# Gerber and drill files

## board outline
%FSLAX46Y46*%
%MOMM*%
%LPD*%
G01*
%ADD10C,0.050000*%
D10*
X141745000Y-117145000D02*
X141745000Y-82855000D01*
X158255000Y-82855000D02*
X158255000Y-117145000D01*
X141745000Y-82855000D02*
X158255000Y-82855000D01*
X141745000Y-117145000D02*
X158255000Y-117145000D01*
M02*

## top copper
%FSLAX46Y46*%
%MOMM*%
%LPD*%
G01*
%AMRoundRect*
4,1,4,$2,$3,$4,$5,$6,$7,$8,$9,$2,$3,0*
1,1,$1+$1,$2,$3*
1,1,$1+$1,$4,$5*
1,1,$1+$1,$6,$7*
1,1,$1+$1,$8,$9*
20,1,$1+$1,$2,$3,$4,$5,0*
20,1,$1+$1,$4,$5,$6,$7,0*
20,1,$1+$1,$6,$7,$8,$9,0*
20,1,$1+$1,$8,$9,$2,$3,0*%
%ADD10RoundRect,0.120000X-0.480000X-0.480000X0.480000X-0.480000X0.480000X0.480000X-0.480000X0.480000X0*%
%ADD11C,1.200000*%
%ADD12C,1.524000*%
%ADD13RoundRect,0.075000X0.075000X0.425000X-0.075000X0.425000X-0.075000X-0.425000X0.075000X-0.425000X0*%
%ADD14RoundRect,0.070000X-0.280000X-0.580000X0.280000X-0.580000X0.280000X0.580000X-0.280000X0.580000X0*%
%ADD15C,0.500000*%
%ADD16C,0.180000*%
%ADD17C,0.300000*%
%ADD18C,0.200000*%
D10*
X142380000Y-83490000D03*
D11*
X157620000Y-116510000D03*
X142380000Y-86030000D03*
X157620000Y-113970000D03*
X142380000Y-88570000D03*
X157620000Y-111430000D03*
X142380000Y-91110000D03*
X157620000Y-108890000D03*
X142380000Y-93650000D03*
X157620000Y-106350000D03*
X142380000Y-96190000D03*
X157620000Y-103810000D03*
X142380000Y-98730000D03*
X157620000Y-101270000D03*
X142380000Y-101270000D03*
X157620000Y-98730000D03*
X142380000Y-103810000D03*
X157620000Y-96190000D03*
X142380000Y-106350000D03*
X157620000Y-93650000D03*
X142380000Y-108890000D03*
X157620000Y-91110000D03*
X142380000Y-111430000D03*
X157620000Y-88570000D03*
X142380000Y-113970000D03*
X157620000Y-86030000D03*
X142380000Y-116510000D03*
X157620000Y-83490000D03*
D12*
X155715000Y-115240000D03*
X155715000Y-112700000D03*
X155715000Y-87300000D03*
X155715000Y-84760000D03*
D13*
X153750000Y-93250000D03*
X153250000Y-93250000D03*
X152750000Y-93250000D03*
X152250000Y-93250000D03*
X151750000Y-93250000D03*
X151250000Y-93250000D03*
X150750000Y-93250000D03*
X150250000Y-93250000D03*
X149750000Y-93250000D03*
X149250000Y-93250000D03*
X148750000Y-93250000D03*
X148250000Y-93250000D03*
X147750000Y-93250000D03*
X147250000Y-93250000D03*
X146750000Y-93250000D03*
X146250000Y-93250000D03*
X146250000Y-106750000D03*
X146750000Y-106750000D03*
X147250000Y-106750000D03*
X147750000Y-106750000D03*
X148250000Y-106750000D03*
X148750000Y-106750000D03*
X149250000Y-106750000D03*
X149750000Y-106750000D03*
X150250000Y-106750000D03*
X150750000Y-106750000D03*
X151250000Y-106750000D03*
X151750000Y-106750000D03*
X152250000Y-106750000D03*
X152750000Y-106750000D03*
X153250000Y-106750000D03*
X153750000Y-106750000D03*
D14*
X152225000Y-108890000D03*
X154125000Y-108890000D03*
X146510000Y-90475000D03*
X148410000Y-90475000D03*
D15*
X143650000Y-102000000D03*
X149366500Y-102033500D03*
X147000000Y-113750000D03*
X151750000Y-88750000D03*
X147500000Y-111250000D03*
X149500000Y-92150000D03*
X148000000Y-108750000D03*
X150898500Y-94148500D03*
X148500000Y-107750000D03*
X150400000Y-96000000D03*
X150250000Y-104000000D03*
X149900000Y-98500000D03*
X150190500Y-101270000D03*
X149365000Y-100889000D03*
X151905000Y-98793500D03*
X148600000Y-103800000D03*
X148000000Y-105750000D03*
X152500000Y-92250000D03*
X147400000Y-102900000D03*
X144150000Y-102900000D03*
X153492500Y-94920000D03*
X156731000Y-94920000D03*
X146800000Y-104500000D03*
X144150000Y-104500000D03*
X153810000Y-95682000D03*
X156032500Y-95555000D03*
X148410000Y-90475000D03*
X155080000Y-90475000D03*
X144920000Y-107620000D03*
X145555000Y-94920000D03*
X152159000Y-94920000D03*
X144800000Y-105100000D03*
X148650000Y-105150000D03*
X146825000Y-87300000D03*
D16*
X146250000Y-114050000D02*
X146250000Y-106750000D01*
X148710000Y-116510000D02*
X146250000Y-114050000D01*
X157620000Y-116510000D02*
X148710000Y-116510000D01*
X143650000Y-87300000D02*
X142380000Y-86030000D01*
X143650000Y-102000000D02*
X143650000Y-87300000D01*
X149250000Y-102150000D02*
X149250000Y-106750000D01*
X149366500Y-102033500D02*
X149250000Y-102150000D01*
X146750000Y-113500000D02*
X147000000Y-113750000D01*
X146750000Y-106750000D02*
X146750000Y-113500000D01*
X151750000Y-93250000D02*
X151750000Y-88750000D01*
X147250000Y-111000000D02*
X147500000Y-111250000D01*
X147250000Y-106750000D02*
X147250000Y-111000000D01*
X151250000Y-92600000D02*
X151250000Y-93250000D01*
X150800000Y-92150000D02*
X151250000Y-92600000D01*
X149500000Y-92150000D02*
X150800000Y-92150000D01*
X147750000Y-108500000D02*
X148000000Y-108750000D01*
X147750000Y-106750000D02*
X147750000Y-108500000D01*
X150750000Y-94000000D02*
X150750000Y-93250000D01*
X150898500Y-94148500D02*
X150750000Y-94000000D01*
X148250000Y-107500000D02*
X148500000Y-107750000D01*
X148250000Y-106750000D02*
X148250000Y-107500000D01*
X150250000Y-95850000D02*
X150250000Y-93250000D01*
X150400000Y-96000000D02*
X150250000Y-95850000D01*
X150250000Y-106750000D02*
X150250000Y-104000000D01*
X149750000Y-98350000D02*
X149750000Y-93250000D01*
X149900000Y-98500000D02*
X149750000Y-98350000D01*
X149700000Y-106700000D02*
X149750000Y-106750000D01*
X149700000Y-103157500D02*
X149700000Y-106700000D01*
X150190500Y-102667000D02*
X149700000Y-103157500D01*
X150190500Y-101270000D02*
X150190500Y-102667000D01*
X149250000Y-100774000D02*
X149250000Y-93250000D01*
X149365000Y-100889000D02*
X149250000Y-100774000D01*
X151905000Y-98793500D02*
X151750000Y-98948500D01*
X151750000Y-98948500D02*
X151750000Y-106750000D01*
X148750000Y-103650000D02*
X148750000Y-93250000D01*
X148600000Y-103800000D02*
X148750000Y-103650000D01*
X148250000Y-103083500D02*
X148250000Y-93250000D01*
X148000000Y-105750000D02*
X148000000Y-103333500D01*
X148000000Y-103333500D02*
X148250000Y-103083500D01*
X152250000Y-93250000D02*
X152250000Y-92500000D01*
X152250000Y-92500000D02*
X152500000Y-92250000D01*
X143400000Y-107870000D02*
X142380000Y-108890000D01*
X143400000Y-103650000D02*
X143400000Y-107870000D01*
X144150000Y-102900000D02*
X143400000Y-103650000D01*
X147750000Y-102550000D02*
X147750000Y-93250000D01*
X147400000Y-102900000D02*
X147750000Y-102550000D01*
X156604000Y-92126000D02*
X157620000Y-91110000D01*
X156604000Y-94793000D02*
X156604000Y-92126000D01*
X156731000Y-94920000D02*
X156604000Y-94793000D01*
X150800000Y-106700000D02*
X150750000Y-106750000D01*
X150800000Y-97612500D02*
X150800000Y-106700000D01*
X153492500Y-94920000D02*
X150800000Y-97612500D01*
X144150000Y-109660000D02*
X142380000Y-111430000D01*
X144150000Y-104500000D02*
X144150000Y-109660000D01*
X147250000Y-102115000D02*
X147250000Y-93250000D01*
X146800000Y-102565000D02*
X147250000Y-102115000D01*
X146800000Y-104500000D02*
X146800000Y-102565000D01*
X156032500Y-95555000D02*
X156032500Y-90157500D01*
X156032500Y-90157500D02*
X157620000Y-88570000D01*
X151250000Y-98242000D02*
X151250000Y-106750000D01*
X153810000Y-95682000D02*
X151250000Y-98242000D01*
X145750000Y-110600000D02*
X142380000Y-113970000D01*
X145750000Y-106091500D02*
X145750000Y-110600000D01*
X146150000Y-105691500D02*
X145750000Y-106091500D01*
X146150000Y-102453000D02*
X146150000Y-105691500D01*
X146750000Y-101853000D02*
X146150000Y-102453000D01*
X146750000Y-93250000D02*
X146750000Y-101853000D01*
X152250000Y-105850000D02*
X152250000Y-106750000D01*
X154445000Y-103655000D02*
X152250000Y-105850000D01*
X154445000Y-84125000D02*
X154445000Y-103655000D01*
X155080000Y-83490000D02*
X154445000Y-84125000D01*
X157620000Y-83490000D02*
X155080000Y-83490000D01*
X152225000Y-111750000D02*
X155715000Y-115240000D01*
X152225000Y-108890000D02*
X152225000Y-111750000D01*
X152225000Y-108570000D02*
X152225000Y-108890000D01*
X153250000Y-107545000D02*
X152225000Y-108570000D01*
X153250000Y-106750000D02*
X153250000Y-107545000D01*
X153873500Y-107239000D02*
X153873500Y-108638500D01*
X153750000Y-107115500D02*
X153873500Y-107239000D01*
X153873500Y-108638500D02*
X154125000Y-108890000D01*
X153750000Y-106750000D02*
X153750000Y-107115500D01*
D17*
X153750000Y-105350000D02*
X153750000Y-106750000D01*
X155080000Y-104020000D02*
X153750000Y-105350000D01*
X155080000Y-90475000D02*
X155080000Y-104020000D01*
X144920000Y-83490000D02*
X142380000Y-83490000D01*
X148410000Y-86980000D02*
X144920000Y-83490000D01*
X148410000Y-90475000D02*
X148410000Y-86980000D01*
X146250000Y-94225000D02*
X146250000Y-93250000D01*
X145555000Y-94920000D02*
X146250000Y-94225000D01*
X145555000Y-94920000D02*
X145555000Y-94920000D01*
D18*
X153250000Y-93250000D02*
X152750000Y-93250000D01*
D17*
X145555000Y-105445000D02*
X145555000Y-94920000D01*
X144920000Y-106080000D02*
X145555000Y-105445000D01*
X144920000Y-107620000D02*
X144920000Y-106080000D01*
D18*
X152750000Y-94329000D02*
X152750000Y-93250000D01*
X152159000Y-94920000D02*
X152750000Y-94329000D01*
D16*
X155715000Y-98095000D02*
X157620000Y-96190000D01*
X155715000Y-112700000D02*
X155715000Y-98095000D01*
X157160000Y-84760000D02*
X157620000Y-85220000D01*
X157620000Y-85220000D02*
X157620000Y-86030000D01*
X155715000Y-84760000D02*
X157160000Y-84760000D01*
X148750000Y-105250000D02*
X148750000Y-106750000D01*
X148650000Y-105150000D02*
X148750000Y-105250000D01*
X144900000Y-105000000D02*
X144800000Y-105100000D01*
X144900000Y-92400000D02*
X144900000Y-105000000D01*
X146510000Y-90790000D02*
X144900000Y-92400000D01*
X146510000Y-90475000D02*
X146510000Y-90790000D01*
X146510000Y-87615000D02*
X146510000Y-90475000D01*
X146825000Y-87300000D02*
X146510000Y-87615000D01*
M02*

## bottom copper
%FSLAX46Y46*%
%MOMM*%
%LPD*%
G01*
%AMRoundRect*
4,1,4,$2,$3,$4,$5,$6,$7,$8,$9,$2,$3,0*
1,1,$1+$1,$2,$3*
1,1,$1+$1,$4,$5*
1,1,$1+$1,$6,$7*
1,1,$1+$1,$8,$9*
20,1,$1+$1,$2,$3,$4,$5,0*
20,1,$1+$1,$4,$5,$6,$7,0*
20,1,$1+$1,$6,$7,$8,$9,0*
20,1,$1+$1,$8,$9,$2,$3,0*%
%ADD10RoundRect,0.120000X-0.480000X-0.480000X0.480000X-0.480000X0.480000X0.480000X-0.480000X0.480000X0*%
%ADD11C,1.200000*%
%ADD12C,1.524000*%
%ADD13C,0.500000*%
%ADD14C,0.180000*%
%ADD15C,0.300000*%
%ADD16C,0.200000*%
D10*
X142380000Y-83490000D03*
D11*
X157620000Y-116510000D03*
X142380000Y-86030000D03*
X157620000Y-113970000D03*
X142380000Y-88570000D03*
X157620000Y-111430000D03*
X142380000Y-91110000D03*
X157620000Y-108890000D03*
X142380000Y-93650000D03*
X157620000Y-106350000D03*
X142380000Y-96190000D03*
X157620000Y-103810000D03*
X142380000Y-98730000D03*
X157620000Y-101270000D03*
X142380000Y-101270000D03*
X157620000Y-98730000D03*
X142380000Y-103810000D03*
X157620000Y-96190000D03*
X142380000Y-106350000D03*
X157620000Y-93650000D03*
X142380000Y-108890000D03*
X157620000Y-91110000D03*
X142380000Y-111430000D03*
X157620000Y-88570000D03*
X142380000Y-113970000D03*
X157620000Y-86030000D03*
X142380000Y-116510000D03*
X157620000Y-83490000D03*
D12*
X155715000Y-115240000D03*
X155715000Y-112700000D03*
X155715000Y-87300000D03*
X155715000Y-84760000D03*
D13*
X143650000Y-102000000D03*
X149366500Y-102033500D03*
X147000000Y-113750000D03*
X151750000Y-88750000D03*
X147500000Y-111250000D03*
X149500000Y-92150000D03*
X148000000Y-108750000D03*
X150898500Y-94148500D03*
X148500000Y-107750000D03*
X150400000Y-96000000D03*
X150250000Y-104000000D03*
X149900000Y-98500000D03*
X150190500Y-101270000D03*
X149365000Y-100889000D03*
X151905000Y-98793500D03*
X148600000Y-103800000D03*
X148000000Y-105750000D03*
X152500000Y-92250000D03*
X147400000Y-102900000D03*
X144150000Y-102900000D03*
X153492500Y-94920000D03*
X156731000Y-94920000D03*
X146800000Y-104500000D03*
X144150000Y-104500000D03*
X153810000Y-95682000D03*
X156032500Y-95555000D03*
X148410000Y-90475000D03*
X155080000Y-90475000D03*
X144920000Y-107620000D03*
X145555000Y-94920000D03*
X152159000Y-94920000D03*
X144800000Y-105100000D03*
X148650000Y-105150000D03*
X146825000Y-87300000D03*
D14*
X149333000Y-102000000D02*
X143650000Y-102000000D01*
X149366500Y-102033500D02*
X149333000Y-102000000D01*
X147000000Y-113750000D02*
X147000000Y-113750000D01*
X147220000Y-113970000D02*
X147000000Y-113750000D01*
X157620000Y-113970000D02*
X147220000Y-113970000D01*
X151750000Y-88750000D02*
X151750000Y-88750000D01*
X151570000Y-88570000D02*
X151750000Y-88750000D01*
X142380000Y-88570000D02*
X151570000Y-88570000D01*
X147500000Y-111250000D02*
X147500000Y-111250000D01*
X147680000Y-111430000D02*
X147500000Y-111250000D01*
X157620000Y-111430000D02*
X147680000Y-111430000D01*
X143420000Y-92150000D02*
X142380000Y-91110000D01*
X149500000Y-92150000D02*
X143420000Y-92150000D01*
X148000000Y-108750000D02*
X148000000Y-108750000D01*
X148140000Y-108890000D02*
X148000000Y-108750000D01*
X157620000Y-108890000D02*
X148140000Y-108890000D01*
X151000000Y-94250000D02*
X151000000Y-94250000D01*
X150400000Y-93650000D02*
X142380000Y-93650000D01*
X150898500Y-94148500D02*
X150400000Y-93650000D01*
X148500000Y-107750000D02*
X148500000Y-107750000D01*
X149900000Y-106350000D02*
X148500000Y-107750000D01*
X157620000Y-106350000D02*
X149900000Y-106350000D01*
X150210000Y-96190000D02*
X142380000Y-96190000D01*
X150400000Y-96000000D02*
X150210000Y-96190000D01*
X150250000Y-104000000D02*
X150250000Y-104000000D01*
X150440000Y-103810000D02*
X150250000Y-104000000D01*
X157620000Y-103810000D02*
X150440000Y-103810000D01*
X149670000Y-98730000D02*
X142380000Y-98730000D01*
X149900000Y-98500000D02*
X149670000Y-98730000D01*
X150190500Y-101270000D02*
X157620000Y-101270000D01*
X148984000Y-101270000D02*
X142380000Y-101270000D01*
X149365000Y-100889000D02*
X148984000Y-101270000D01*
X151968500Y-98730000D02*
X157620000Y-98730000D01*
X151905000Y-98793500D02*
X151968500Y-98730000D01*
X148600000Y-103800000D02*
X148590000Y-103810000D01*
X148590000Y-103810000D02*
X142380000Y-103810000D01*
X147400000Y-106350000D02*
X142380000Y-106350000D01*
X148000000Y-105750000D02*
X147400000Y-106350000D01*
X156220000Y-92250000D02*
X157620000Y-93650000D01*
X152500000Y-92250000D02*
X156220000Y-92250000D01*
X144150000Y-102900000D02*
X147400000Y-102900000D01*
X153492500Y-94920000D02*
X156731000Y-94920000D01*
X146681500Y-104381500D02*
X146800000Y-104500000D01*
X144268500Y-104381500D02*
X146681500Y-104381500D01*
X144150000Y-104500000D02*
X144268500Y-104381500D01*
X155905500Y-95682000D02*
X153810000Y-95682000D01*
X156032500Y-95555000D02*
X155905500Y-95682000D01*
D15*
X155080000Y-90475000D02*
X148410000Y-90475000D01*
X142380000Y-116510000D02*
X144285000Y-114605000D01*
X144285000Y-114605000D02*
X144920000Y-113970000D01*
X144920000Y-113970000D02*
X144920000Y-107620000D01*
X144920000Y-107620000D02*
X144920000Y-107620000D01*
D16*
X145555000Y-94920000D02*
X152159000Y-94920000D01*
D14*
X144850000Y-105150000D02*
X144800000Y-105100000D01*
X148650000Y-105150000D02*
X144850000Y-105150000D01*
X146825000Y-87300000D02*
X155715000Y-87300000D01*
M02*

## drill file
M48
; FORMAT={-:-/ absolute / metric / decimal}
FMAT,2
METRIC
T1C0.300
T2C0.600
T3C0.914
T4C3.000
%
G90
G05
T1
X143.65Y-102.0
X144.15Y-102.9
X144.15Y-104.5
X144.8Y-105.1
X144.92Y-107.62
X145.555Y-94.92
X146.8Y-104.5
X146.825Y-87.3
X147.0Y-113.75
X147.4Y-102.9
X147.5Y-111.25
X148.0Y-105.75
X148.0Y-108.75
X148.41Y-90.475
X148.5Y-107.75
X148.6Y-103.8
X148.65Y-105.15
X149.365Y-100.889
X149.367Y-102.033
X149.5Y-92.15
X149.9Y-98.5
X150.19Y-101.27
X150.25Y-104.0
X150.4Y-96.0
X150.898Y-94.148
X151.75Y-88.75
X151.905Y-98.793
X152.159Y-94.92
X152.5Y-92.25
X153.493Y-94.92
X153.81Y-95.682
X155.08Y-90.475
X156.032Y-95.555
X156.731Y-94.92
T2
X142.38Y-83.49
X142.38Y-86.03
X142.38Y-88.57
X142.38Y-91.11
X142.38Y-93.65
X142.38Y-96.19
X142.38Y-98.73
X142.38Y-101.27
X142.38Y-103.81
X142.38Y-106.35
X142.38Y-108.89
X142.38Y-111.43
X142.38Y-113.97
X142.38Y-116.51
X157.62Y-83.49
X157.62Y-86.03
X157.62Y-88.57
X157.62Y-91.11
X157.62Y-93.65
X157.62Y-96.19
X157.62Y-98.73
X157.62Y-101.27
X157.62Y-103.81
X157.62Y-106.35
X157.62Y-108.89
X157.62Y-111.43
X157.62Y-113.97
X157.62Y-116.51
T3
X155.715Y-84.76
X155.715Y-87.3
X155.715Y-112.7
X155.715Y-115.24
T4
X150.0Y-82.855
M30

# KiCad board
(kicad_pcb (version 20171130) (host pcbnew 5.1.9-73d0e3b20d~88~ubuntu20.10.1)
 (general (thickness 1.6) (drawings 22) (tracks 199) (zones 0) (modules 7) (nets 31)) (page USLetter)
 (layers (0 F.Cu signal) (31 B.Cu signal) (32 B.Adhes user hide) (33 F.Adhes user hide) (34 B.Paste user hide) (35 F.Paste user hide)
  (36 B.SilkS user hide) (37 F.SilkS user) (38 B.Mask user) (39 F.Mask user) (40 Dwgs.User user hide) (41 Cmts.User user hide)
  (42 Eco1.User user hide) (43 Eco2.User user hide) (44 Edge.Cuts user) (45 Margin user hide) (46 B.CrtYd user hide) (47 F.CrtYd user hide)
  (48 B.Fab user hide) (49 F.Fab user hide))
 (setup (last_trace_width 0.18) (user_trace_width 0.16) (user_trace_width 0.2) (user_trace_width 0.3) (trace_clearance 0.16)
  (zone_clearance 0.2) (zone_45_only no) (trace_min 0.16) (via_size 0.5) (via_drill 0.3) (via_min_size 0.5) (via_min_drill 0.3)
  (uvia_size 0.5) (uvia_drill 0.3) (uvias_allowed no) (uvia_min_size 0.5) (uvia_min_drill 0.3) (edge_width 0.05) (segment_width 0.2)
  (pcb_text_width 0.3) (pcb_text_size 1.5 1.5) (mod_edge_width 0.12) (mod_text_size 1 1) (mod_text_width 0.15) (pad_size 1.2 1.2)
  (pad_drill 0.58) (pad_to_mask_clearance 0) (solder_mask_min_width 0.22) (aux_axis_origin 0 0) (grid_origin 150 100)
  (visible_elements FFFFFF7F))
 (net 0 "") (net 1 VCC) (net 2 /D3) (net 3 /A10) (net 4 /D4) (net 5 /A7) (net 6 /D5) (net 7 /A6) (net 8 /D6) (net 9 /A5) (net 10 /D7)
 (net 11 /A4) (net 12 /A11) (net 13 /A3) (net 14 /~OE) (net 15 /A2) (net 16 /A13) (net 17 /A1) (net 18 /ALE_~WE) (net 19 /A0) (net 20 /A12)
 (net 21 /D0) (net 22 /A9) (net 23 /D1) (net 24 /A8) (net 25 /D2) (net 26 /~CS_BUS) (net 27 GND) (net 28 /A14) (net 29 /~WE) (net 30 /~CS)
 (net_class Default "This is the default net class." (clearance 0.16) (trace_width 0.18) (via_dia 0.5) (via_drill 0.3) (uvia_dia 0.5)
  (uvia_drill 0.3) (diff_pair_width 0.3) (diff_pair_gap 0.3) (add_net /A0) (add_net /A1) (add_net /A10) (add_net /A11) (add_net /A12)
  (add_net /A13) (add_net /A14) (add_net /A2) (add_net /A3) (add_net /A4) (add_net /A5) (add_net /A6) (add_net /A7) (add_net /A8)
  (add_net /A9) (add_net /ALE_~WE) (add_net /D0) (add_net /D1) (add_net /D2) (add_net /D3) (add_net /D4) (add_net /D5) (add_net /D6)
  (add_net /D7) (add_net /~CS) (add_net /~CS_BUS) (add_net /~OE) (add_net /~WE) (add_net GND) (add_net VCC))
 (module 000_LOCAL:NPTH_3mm (layer F.Cu) (at 150 82.855)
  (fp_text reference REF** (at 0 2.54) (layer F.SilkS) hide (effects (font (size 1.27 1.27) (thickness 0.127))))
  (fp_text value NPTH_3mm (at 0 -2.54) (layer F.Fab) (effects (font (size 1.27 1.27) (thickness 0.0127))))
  (pad "" np_thru_hole circle (at 0 0) (size 3 3) (drill 3) (layers *.Cu *.Mask)))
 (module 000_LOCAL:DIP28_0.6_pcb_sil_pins (layer F.Cu) (at 150 100)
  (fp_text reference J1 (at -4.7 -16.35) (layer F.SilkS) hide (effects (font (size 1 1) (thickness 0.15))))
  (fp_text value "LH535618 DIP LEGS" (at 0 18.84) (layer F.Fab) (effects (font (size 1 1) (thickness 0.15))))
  (pad 1 thru_hole roundrect (at -7.62 -16.51) (size 1.2 1.2) (drill 0.6) (layers *.Cu *.Mask) (roundrect_rratio 0.1) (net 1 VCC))
  (pad 15 thru_hole circle (at 7.62 16.51) (size 1.2 1.2) (drill 0.6) (layers *.Cu *.Mask) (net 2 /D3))
  (pad 2 thru_hole circle (at -7.62 -13.97) (size 1.2 1.2) (drill 0.6) (layers *.Cu *.Mask) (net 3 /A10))
  (pad 16 thru_hole circle (at 7.62 13.97) (size 1.2 1.2) (drill 0.6) (layers *.Cu *.Mask) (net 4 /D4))
  (pad 3 thru_hole circle (at -7.62 -11.43) (size 1.2 1.2) (drill 0.6) (layers *.Cu *.Mask) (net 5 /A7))
  (pad 17 thru_hole circle (at 7.62 11.43) (size 1.2 1.2) (drill 0.6) (layers *.Cu *.Mask) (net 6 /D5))
  (pad 4 thru_hole circle (at -7.62 -8.89) (size 1.2 1.2) (drill 0.6) (layers *.Cu *.Mask) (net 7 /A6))
  (pad 18 thru_hole circle (at 7.62 8.89) (size 1.2 1.2) (drill 0.6) (layers *.Cu *.Mask) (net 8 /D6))
  (pad 5 thru_hole circle (at -7.62 -6.35) (size 1.2 1.2) (drill 0.6) (layers *.Cu *.Mask) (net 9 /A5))
  (pad 19 thru_hole circle (at 7.62 6.35) (size 1.2 1.2) (drill 0.6) (layers *.Cu *.Mask) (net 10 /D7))
  (pad 6 thru_hole circle (at -7.62 -3.81) (size 1.2 1.2) (drill 0.6) (layers *.Cu *.Mask) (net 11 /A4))
  (pad 20 thru_hole circle (at 7.62 3.81) (size 1.2 1.2) (drill 0.6) (layers *.Cu *.Mask) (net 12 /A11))
  (pad 7 thru_hole circle (at -7.62 -1.27) (size 1.2 1.2) (drill 0.6) (layers *.Cu *.Mask) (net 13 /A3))
  (pad 21 thru_hole circle (at 7.62 1.27) (size 1.2 1.2) (drill 0.6) (layers *.Cu *.Mask) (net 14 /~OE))
  (pad 8 thru_hole circle (at -7.62 1.27) (size 1.2 1.2) (drill 0.6) (layers *.Cu *.Mask) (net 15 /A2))
  (pad 22 thru_hole circle (at 7.62 -1.27) (size 1.2 1.2) (drill 0.6) (layers *.Cu *.Mask) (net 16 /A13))
  (pad 9 thru_hole circle (at -7.62 3.81) (size 1.2 1.2) (drill 0.6) (layers *.Cu *.Mask) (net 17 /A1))
  (pad 23 thru_hole circle (at 7.62 -3.81) (size 1.2 1.2) (drill 0.6) (layers *.Cu *.Mask) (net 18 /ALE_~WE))
  (pad 10 thru_hole circle (at -7.62 6.35) (size 1.2 1.2) (drill 0.6) (layers *.Cu *.Mask) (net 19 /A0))
  (pad 24 thru_hole circle (at 7.62 -6.35) (size 1.2 1.2) (drill 0.6) (layers *.Cu *.Mask) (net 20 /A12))
  (pad 11 thru_hole circle (at -7.62 8.89) (size 1.2 1.2) (drill 0.6) (layers *.Cu *.Mask) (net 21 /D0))
  (pad 25 thru_hole circle (at 7.62 -8.89) (size 1.2 1.2) (drill 0.6) (layers *.Cu *.Mask) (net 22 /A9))
  (pad 12 thru_hole circle (at -7.62 11.43) (size 1.2 1.2) (drill 0.6) (layers *.Cu *.Mask) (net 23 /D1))
  (pad 26 thru_hole circle (at 7.62 -11.43) (size 1.2 1.2) (drill 0.6) (layers *.Cu *.Mask) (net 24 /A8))
  (pad 13 thru_hole circle (at -7.62 13.97) (size 1.2 1.2) (drill 0.6) (layers *.Cu *.Mask) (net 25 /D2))
  (pad 27 thru_hole circle (at 7.62 -13.97) (size 1.2 1.2) (drill 0.6) (layers *.Cu *.Mask) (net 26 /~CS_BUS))
  (pad 14 thru_hole circle (at -7.62 16.51) (size 1.2 1.2) (drill 0.6) (layers *.Cu *.Mask) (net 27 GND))
  (pad 28 thru_hole circle (at 7.62 -16.51) (size 1.2 1.2) (drill 0.6) (layers *.Cu *.Mask) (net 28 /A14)))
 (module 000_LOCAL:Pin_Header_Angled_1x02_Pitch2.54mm (layer F.Cu) (at 155.715 115.24 180)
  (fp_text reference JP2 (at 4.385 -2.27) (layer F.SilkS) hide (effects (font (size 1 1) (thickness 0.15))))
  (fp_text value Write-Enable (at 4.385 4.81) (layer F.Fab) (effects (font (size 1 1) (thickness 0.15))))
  (pad 1 thru_hole circle (at 0 0 180) (size 1.524 1.524) (drill 0.9144) (layers *.Cu *.Mask) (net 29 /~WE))
  (pad 2 thru_hole circle (at 0 2.54 180) (size 1.524 1.524) (drill 0.9144) (layers *.Cu *.Mask) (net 18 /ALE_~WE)))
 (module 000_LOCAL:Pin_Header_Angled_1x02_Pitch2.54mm (layer F.Cu) (at 155.715 87.3 180)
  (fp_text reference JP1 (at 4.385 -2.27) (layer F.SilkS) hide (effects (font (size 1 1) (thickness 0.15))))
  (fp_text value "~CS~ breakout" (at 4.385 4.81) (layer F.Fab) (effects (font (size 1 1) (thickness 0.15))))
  (pad 1 thru_hole circle (at 0 0 180) (size 1.524 1.524) (drill 0.9144) (layers *.Cu *.Mask) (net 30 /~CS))
  (pad 2 thru_hole circle (at 0 2.54 180) (size 1.524 1.524) (drill 0.9144) (layers *.Cu *.Mask) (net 26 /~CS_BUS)))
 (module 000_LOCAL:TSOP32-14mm (layer F.Cu) (at 150 100 180)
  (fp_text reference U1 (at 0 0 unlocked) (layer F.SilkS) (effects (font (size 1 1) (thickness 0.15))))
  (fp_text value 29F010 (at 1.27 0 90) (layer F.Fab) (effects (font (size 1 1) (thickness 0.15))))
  (pad 1 smd roundrect (at -3.75 6.75 180) (size 0.3 1) (layers F.Cu F.Paste F.Mask) (roundrect_rratio 0.25))
  (pad 2 smd roundrect (at -3.25 6.75 180) (size 0.3 1) (layers F.Cu F.Paste F.Mask) (roundrect_rratio 0.25) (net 27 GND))
  (pad 3 smd roundrect (at -2.75 6.75 180) (size 0.3 1) (layers F.Cu F.Paste F.Mask) (roundrect_rratio 0.25) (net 27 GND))
  (pad 4 smd roundrect (at -2.25 6.75 180) (size 0.3 1) (layers F.Cu F.Paste F.Mask) (roundrect_rratio 0.25) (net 20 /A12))
  (pad 5 smd roundrect (at -1.75 6.75 180) (size 0.3 1) (layers F.Cu F.Paste F.Mask) (roundrect_rratio 0.25) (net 5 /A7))
  (pad 6 smd roundrect (at -1.25 6.75 180) (size 0.3 1) (layers F.Cu F.Paste F.Mask) (roundrect_rratio 0.25) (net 7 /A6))
  (pad 7 smd roundrect (at -0.75 6.75 180) (size 0.3 1) (layers F.Cu F.Paste F.Mask) (roundrect_rratio 0.25) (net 9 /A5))
  (pad 8 smd roundrect (at -0.25 6.75 180) (size 0.3 1) (layers F.Cu F.Paste F.Mask) (roundrect_rratio 0.25) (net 11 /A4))
  (pad 9 smd roundrect (at 0.25 6.75 180) (size 0.3 1) (layers F.Cu F.Paste F.Mask) (roundrect_rratio 0.25) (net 13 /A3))
  (pad 10 smd roundrect (at 0.75 6.75 180) (size 0.3 1) (layers F.Cu F.Paste F.Mask) (roundrect_rratio 0.25) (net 15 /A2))
  (pad 11 smd roundrect (at 1.25 6.75 180) (size 0.3 1) (layers F.Cu F.Paste F.Mask) (roundrect_rratio 0.25) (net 17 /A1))
  (pad 12 smd roundrect (at 1.75 6.75 180) (size 0.3 1) (layers F.Cu F.Paste F.Mask) (roundrect_rratio 0.25) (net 19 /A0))
  (pad 13 smd roundrect (at 2.25 6.75 180) (size 0.3 1) (layers F.Cu F.Paste F.Mask) (roundrect_rratio 0.25) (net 21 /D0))
  (pad 14 smd roundrect (at 2.75 6.75 180) (size 0.3 1) (layers F.Cu F.Paste F.Mask) (roundrect_rratio 0.25) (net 23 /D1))
  (pad 15 smd roundrect (at 3.25 6.75 180) (size 0.3 1) (layers F.Cu F.Paste F.Mask) (roundrect_rratio 0.25) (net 25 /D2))
  (pad 16 smd roundrect (at 3.75 6.75 180) (size 0.3 1) (layers F.Cu F.Paste F.Mask) (roundrect_rratio 0.25) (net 27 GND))
  (pad 17 smd roundrect (at 3.75 -6.75 180) (size 0.3 1) (layers F.Cu F.Paste F.Mask) (roundrect_rratio 0.25) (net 2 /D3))
  (pad 18 smd roundrect (at 3.25 -6.75 180) (size 0.3 1) (layers F.Cu F.Paste F.Mask) (roundrect_rratio 0.25) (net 4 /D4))
  (pad 19 smd roundrect (at 2.75 -6.75 180) (size 0.3 1) (layers F.Cu F.Paste F.Mask) (roundrect_rratio 0.25) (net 6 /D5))
  (pad 20 smd roundrect (at 2.25 -6.75 180) (size 0.3 1) (layers F.Cu F.Paste F.Mask) (roundrect_rratio 0.25) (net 8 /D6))
  (pad 21 smd roundrect (at 1.75 -6.75 180) (size 0.3 1) (layers F.Cu F.Paste F.Mask) (roundrect_rratio 0.25) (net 10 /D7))
  (pad 22 smd roundrect (at 1.25 -6.75 180) (size 0.3 1) (layers F.Cu F.Paste F.Mask) (roundrect_rratio 0.25) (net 30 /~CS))
  (pad 23 smd roundrect (at 0.75 -6.75 180) (size 0.3 1) (layers F.Cu F.Paste F.Mask) (roundrect_rratio 0.25) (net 3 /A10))
  (pad 24 smd roundrect (at 0.25 -6.75 180) (size 0.3 1) (layers F.Cu F.Paste F.Mask) (roundrect_rratio 0.25) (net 14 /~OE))
  (pad 25 smd roundrect (at -0.25 -6.75 180) (size 0.3 1) (layers F.Cu F.Paste F.Mask) (roundrect_rratio 0.25) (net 12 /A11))
  (pad 26 smd roundrect (at -0.75 -6.75 180) (size 0.3 1) (layers F.Cu F.Paste F.Mask) (roundrect_rratio 0.25) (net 22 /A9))
  (pad 27 smd roundrect (at -1.25 -6.75 180) (size 0.3 1) (layers F.Cu F.Paste F.Mask) (roundrect_rratio 0.25) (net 24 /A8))
  (pad 28 smd roundrect (at -1.75 -6.75 180) (size 0.3 1) (layers F.Cu F.Paste F.Mask) (roundrect_rratio 0.25) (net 16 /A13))
  (pad 29 smd roundrect (at -2.25 -6.75 180) (size 0.3 1) (layers F.Cu F.Paste F.Mask) (roundrect_rratio 0.25) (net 28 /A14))
  (pad 30 smd roundrect (at -2.75 -6.75 180) (size 0.3 1) (layers F.Cu F.Paste F.Mask) (roundrect_rratio 0.25))
  (pad 31 smd roundrect (at -3.25 -6.75 180) (size 0.3 1) (layers F.Cu F.Paste F.Mask) (roundrect_rratio 0.25) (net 29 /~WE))
  (pad 32 smd roundrect (at -3.75 -6.75 180) (size 0.3 1) (layers F.Cu F.Paste F.Mask) (roundrect_rratio 0.25) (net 1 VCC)))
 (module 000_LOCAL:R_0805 (layer F.Cu) (at 153.175 108.89)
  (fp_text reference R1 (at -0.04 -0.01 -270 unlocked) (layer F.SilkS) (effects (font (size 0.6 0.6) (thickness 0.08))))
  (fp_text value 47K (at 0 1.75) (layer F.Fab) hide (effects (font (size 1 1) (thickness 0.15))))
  (pad 1 smd roundrect (at -0.95 0) (size 0.7 1.3) (layers F.Cu F.Paste F.Mask) (roundrect_rratio 0.1) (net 29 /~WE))
  (pad 2 smd roundrect (at 0.95 0) (size 0.7 1.3) (layers F.Cu F.Paste F.Mask) (roundrect_rratio 0.1) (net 1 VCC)))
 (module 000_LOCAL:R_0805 (layer F.Cu) (at 147.46 90.475)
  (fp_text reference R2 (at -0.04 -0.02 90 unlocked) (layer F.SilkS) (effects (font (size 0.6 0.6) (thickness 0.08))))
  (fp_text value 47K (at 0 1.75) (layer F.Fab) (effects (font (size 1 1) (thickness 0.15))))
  (pad 1 smd roundrect (at -0.95 0) (size 0.7 1.3) (layers F.Cu F.Paste F.Mask) (roundrect_rratio 0.1) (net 30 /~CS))
  (pad 2 smd roundrect (at 0.95 0) (size 0.7 1.3) (layers F.Cu F.Paste F.Mask) (roundrect_rratio 0.1) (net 1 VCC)))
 (gr_line (start 141.745 117.145) (end 141.745 82.855) (layer Edge.Cuts) (width 0.05))
 (gr_line (start 158.255 82.855) (end 158.255 117.145) (layer Edge.Cuts) (width 0.05))
 (gr_line (start 141.745 82.855) (end 158.255 82.855) (layer Edge.Cuts) (width 0.05))
 (gr_line (start 141.745 117.145) (end 158.255 117.145) (layer Edge.Cuts) (width 0.05))
 (segment (start 146.25 114.05) (end 146.25 106.75) (width 0.18) (layer F.Cu) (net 2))
 (segment (start 148.71 116.51) (end 146.25 114.05) (width 0.18) (layer F.Cu) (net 2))
 (segment (start 157.62 116.51) (end 148.71 116.51) (width 0.18) (layer F.Cu) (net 2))
 (segment (start 143.65 87.3) (end 142.38 86.03) (width 0.18) (layer F.Cu) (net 3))
 (segment (start 143.65 102) (end 143.65 87.3) (width 0.18) (layer F.Cu) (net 3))
 (via (at 143.65 102) (size 0.5) (drill 0.3) (layers F.Cu B.Cu) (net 3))
 (segment (start 149.333 102) (end 143.65 102) (width 0.18) (layer B.Cu) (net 3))
 (segment (start 149.3665 102.0335) (end 149.333 102) (width 0.18) (layer B.Cu) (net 3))
 (segment (start 149.25 102.15) (end 149.25 106.75) (width 0.18) (layer F.Cu) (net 3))
 (segment (start 149.3665 102.0335) (end 149.25 102.15) (width 0.18) (layer F.Cu) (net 3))
 (via (at 149.3665 102.0335) (size 0.5) (drill 0.3) (layers F.Cu B.Cu) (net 3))
 (segment (start 147 113.75) (end 147 113.75) (width 0.18) (layer B.Cu) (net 4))
 (via (at 147 113.75) (size 0.5) (drill 0.3) (layers F.Cu B.Cu) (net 4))
 (segment (start 146.75 113.5) (end 147 113.75) (width 0.18) (layer F.Cu) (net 4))
 (segment (start 146.75 106.75) (end 146.75 113.5) (width 0.18) (layer F.Cu) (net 4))
 (segment (start 147.22 113.97) (end 147 113.75) (width 0.18) (layer B.Cu) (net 4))
 (segment (start 157.62 113.97) (end 147.22 113.97) (width 0.18) (layer B.Cu) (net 4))
 (segment (start 151.75 88.75) (end 151.75 88.75) (width 0.18) (layer B.Cu) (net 5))
 (via (at 151.75 88.75) (size 0.5) (drill 0.3) (layers F.Cu B.Cu) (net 5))
 (segment (start 151.75 93.25) (end 151.75 88.75) (width 0.18) (layer F.Cu) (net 5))
 (segment (start 151.57 88.57) (end 151.75 88.75) (width 0.18) (layer B.Cu) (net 5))
 (segment (start 142.38 88.57) (end 151.57 88.57) (width 0.18) (layer B.Cu) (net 5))
 (segment (start 147.5 111.25) (end 147.5 111.25) (width 0.18) (layer B.Cu) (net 6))
 (via (at 147.5 111.25) (size 0.5) (drill 0.3) (layers F.Cu B.Cu) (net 6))
 (segment (start 147.25 111) (end 147.5 111.25) (width 0.18) (layer F.Cu) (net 6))
 (segment (start 147.25 106.75) (end 147.25 111) (width 0.18) (layer F.Cu) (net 6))
 (segment (start 147.68 111.43) (end 147.5 111.25) (width 0.18) (layer B.Cu) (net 6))
 (segment (start 157.62 111.43) (end 147.68 111.43) (width 0.18) (layer B.Cu) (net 6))
 (via (at 149.5 92.15) (size 0.5) (drill 0.3) (layers F.Cu B.Cu) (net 7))
 (segment (start 151.25 92.6) (end 151.25 93.25) (width 0.18) (layer F.Cu) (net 7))
 (segment (start 150.8 92.15) (end 151.25 92.6) (width 0.18) (layer F.Cu) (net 7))
 (segment (start 149.5 92.15) (end 150.8 92.15) (width 0.18) (layer F.Cu) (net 7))
 (segment (start 143.42 92.15) (end 142.38 91.11) (width 0.18) (layer B.Cu) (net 7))
 (segment (start 149.5 92.15) (end 143.42 92.15) (width 0.18) (layer B.Cu) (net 7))
 (segment (start 148 108.75) (end 148 108.75) (width 0.18) (layer B.Cu) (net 8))
 (via (at 148 108.75) (size 0.5) (drill 0.3) (layers F.Cu B.Cu) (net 8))
 (segment (start 147.75 108.5) (end 148 108.75) (width 0.18) (layer F.Cu) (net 8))
 (segment (start 147.75 106.75) (end 147.75 108.5) (width 0.18) (layer F.Cu) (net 8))
 (segment (start 148.14 108.89) (end 148 108.75) (width 0.18) (layer B.Cu) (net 8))
 (segment (start 157.62 108.89) (end 148.14 108.89) (width 0.18) (layer B.Cu) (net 8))
 (segment (start 151 94.25) (end 151 94.25) (width 0.18) (layer B.Cu) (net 9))
 (segment (start 150.4 93.65) (end 142.38 93.65) (width 0.18) (layer B.Cu) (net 9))
 (segment (start 150.8985 94.1485) (end 150.4 93.65) (width 0.18) (layer B.Cu) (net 9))
 (segment (start 150.75 94) (end 150.75 93.25) (width 0.18) (layer F.Cu) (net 9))
 (segment (start 150.8985 94.1485) (end 150.75 94) (width 0.18) (layer F.Cu) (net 9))
 (via (at 150.8985 94.1485) (size 0.5) (drill 0.3) (layers F.Cu B.Cu) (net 9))
 (segment (start 148.5 107.75) (end 148.5 107.75) (width 0.18) (layer B.Cu) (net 10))
 (via (at 148.5 107.75) (size 0.5) (drill 0.3) (layers F.Cu B.Cu) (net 10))
 (segment (start 148.25 107.5) (end 148.5 107.75) (width 0.18) (layer F.Cu) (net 10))
 (segment (start 148.25 106.75) (end 148.25 107.5) (width 0.18) (layer F.Cu) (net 10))
 (segment (start 149.9 106.35) (end 148.5 107.75) (width 0.18) (layer B.Cu) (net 10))
 (segment (start 157.62 106.35) (end 149.9 106.35) (width 0.18) (layer B.Cu) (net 10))
 (segment (start 150.25 95.85) (end 150.25 93.25) (width 0.18) (layer F.Cu) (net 11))
 (segment (start 150.4 96) (end 150.25 95.85) (width 0.18) (layer F.Cu) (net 11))
 (via (at 150.4 96) (size 0.5) (drill 0.3) (layers F.Cu B.Cu) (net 11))
 (segment (start 150.21 96.19) (end 142.38 96.19) (width 0.18) (layer B.Cu) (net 11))
 (segment (start 150.4 96) (end 150.21 96.19) (width 0.18) (layer B.Cu) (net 11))
 (segment (start 150.25 104) (end 150.25 104) (width 0.18) (layer B.Cu) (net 12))
 (via (at 150.25 104) (size 0.5) (drill 0.3) (layers F.Cu B.Cu) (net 12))
 (segment (start 150.25 106.75) (end 150.25 104) (width 0.18) (layer F.Cu) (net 12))
 (segment (start 150.44 103.81) (end 150.25 104) (width 0.18) (layer B.Cu) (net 12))
 (segment (start 157.62 103.81) (end 150.44 103.81) (width 0.18) (layer B.Cu) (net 12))
 (segment (start 149.75 98.35) (end 149.75 93.25) (width 0.18) (layer F.Cu) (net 13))
 (segment (start 149.9 98.5) (end 149.75 98.35) (width 0.18) (layer F.Cu) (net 13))
 (via (at 149.9 98.5) (size 0.5) (drill 0.3) (layers F.Cu B.Cu) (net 13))
 (segment (start 149.67 98.73) (end 142.38 98.73) (width 0.18) (layer B.Cu) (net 13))
 (segment (start 149.9 98.5) (end 149.67 98.73) (width 0.18) (layer B.Cu) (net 13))
 (segment (start 150.1905 101.27) (end 157.62 101.27) (width 0.18) (layer B.Cu) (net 14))
 (via (at 150.1905 101.27) (size 0.5) (drill 0.3) (layers F.Cu B.Cu) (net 14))
 (segment (start 149.7 106.7) (end 149.75 106.75) (width 0.18) (layer F.Cu) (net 14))
 (segment (start 149.7 103.1575) (end 149.7 106.7) (width 0.18) (layer F.Cu) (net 14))
 (segment (start 150.1905 102.667) (end 149.7 103.1575) (width 0.18) (layer F.Cu) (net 14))
 (segment (start 150.1905 101.27) (end 150.1905 102.667) (width 0.18) (layer F.Cu) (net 14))
 (segment (start 149.25 100.774) (end 149.25 93.25) (width 0.18) (layer F.Cu) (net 15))
 (segment (start 149.365 100.889) (end 149.25 100.774) (width 0.18) (layer F.Cu) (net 15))
 (segment (start 148.984 101.27) (end 142.38 101.27) (width 0.18) (layer B.Cu) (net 15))
 (segment (start 149.365 100.889) (end 148.984 101.27) (width 0.18) (layer B.Cu) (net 15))
 (via (at 149.365 100.889) (size 0.5) (drill 0.3) (layers F.Cu B.Cu) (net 15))
 (segment (start 151.905 98.7935) (end 151.75 98.9485) (width 0.18) (layer F.Cu) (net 16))
 (segment (start 151.9685 98.73) (end 157.62 98.73) (width 0.18) (layer B.Cu) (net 16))
 (segment (start 151.75 98.9485) (end 151.75 106.75) (width 0.18) (layer F.Cu) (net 16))
 (segment (start 151.905 98.7935) (end 151.9685 98.73) (width 0.18) (layer B.Cu) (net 16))
 (via (at 151.905 98.7935) (size 0.5) (drill 0.3) (layers F.Cu B.Cu) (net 16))
 (segment (start 148.6 103.8) (end 148.59 103.81) (width 0.18) (layer B.Cu) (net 17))
 (segment (start 148.75 103.65) (end 148.75 93.25) (width 0.18) (layer F.Cu) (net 17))
 (segment (start 148.6 103.8) (end 148.75 103.65) (width 0.18) (layer F.Cu) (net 17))
 (segment (start 148.59 103.81) (end 142.38 103.81) (width 0.18) (layer B.Cu) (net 17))
 (via (at 148.6 103.8) (size 0.5) (drill 0.3) (layers F.Cu B.Cu) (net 17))
 (segment (start 148.25 103.0835) (end 148.25 93.25) (width 0.18) (layer F.Cu) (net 19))
 (segment (start 148 105.75) (end 148 103.3335) (width 0.18) (layer F.Cu) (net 19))
 (segment (start 147.4 106.35) (end 142.38 106.35) (width 0.18) (layer B.Cu) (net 19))
 (segment (start 148 103.3335) (end 148.25 103.0835) (width 0.18) (layer F.Cu) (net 19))
 (segment (start 148 105.75) (end 147.4 106.35) (width 0.18) (layer B.Cu) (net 19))
 (via (at 148 105.75) (size 0.5) (drill 0.3) (layers F.Cu B.Cu) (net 19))
 (segment (start 152.25 93.25) (end 152.25 92.5) (width 0.18) (layer F.Cu) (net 20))
 (segment (start 152.25 92.5) (end 152.5 92.25) (width 0.18) (layer F.Cu) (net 20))
 (via (at 152.5 92.25) (size 0.5) (drill 0.3) (layers F.Cu B.Cu) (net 20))
 (segment (start 156.22 92.25) (end 157.62 93.65) (width 0.18) (layer B.Cu) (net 20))
 (segment (start 152.5 92.25) (end 156.22 92.25) (width 0.18) (layer B.Cu) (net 20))
 (via (at 147.4 102.9) (size 0.5) (drill 0.3) (layers F.Cu B.Cu) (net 21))
 (segment (start 144.15 102.9) (end 147.4 102.9) (width 0.18) (layer B.Cu) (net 21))
 (via (at 144.15 102.9) (size 0.5) (drill 0.3) (layers F.Cu B.Cu) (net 21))
 (segment (start 143.4 107.87) (end 142.38 108.89) (width 0.18) (layer F.Cu) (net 21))
 (segment (start 143.4 103.65) (end 143.4 107.87) (width 0.18) (layer F.Cu) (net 21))
 (segment (start 144.15 102.9) (end 143.4 103.65) (width 0.18) (layer F.Cu) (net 21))
 (segment (start 147.75 102.55) (end 147.75 93.25) (width 0.18) (layer F.Cu) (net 21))
 (segment (start 147.4 102.9) (end 147.75 102.55) (width 0.18) (layer F.Cu) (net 21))
 (via (at 153.4925 94.92) (size 0.5) (drill 0.3) (layers F.Cu B.Cu) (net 22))
 (segment (start 156.604 92.126) (end 157.62 91.11) (width 0.18) (layer F.Cu) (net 22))
 (segment (start 156.604 94.793) (end 156.604 92.126) (width 0.18) (layer F.Cu) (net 22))
 (segment (start 156.731 94.92) (end 156.604 94.793) (width 0.18) (layer F.Cu) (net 22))
 (segment (start 153.4925 94.92) (end 156.731 94.92) (width 0.18) (layer B.Cu) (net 22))
 (via (at 156.731 94.92) (size 0.5) (drill 0.3) (layers F.Cu B.Cu) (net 22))
 (segment (start 150.8 106.7) (end 150.75 106.75) (width 0.18) (layer F.Cu) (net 22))
 (segment (start 150.8 97.6125) (end 150.8 106.7) (width 0.18) (layer F.Cu) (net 22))
 (segment (start 153.4925 94.92) (end 150.8 97.6125) (width 0.18) (layer F.Cu) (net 22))
 (via (at 146.8 104.5) (size 0.5) (drill 0.3) (layers F.Cu B.Cu) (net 23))
 (segment (start 144.15 109.66) (end 142.38 111.43) (width 0.18) (layer F.Cu) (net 23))
 (segment (start 144.15 104.5) (end 144.15 109.66) (width 0.18) (layer F.Cu) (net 23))
 (via (at 144.15 104.5) (size 0.5) (drill 0.3) (layers F.Cu B.Cu) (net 23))
 (segment (start 146.6815 104.3815) (end 146.8 104.5) (width 0.18) (layer B.Cu) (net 23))
 (segment (start 144.2685 104.3815) (end 146.6815 104.3815) (width 0.18) (layer B.Cu) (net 23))
 (segment (start 144.15 104.5) (end 144.2685 104.3815) (width 0.18) (layer B.Cu) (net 23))
 (segment (start 147.25 102.115) (end 147.25 93.25) (width 0.18) (layer F.Cu) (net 23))
 (segment (start 146.8 102.565) (end 147.25 102.115) (width 0.18) (layer F.Cu) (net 23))
 (segment (start 146.8 104.5) (end 146.8 102.565) (width 0.18) (layer F.Cu) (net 23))
 (via (at 153.81 95.682) (size 0.5) (drill 0.3) (layers F.Cu B.Cu) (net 24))
 (segment (start 156.0325 95.555) (end 156.0325 90.1575) (width 0.18) (layer F.Cu) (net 24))
 (segment (start 156.0325 90.1575) (end 157.62 88.57) (width 0.18) (layer F.Cu) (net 24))
 (via (at 156.0325 95.555) (size 0.5) (drill 0.3) (layers F.Cu B.Cu) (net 24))
 (segment (start 151.25 98.242) (end 151.25 106.75) (width 0.18) (layer F.Cu) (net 24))
 (segment (start 153.81 95.682) (end 151.25 98.242) (width 0.18) (layer F.Cu) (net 24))
 (segment (start 155.9055 95.682) (end 153.81 95.682) (width 0.18) (layer B.Cu) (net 24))
 (segment (start 156.0325 95.555) (end 155.9055 95.682) (width 0.18) (layer B.Cu) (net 24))
 (segment (start 145.75 110.6) (end 142.38 113.97) (width 0.18) (layer F.Cu) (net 25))
 (segment (start 145.75 106.0915) (end 145.75 110.6) (width 0.18) (layer F.Cu) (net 25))
 (segment (start 146.15 105.6915) (end 145.75 106.0915) (width 0.18) (layer F.Cu) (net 25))
 (segment (start 146.15 102.453) (end 146.15 105.6915) (width 0.18) (layer F.Cu) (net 25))
 (segment (start 146.75 101.853) (end 146.15 102.453) (width 0.18) (layer F.Cu) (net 25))
 (segment (start 146.75 93.25) (end 146.75 101.853) (width 0.18) (layer F.Cu) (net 25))
 (segment (start 152.25 105.85) (end 152.25 106.75) (width 0.18) (layer F.Cu) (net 28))
 (segment (start 154.445 103.655) (end 152.25 105.85) (width 0.18) (layer F.Cu) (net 28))
 (segment (start 154.445 84.125) (end 154.445 103.655) (width 0.18) (layer F.Cu) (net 28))
 (segment (start 155.08 83.49) (end 154.445 84.125) (width 0.18) (layer F.Cu) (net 28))
 (segment (start 157.62 83.49) (end 155.08 83.49) (width 0.18) (layer F.Cu) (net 28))
 (segment (start 152.225 111.75) (end 155.715 115.24) (width 0.18) (layer F.Cu) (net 29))
 (segment (start 152.225 108.89) (end 152.225 111.75) (width 0.18) (layer F.Cu) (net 29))
 (segment (start 152.225 108.57) (end 152.225 108.89) (width 0.18) (layer F.Cu) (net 29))
 (segment (start 153.25 107.545) (end 152.225 108.57) (width 0.18) (layer F.Cu) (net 29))
 (segment (start 153.25 106.75) (end 153.25 107.545) (width 0.18) (layer F.Cu) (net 29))
 (segment (start 153.8735 107.239) (end 153.8735 108.6385) (width 0.18) (layer F.Cu) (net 1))
 (segment (start 153.75 107.1155) (end 153.8735 107.239) (width 0.18) (layer F.Cu) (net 1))
 (segment (start 153.8735 108.6385) (end 154.125 108.89) (width 0.18) (layer F.Cu) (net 1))
 (segment (start 153.75 106.75) (end 153.75 107.1155) (width 0.18) (layer F.Cu) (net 1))
 (via (at 148.41 90.475) (size 0.5) (drill 0.3) (layers F.Cu B.Cu) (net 1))
 (segment (start 155.08 90.475) (end 148.41 90.475) (width 0.3) (layer B.Cu) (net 1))
 (segment (start 153.75 105.35) (end 153.75 106.75) (width 0.3) (layer F.Cu) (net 1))
 (segment (start 155.08 104.02) (end 153.75 105.35) (width 0.3) (layer F.Cu) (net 1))
 (segment (start 155.08 90.475) (end 155.08 104.02) (width 0.3) (layer F.Cu) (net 1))
 (via (at 155.08 90.475) (size 0.5) (drill 0.3) (layers F.Cu B.Cu) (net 1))
 (segment (start 144.92 83.49) (end 142.38 83.49) (width 0.3) (layer F.Cu) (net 1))
 (segment (start 148.41 86.98) (end 144.92 83.49) (width 0.3) (layer F.Cu) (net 1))
 (segment (start 148.41 90.475) (end 148.41 86.98) (width 0.3) (layer F.Cu) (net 1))
 (segment (start 142.38 116.51) (end 144.285 114.605) (width 0.3) (layer B.Cu) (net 27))
 (segment (start 144.285 114.605) (end 144.92 113.97) (width 0.3) (layer B.Cu) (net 27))
 (segment (start 144.92 113.97) (end 144.92 107.62) (width 0.3) (layer B.Cu) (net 27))
 (segment (start 144.92 107.62) (end 144.92 107.62) (width 0.3) (layer B.Cu) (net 27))
 (via (at 144.92 107.62) (size 0.5) (drill 0.3) (layers F.Cu B.Cu) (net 27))
 (segment (start 146.25 94.225) (end 146.25 93.25) (width 0.3) (layer F.Cu) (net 27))
 (segment (start 145.555 94.92) (end 146.25 94.225) (width 0.3) (layer F.Cu) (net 27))
 (segment (start 145.555 94.92) (end 145.555 94.92) (width 0.3) (layer F.Cu) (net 27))
 (via (at 145.555 94.92) (size 0.5) (drill 0.3) (layers F.Cu B.Cu) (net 27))
 (segment (start 153.25 93.25) (end 152.75 93.25) (width 0.2) (layer F.Cu) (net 27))
 (segment (start 145.555 105.445) (end 145.555 94.92) (width 0.3) (layer F.Cu) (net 27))
 (segment (start 144.92 106.08) (end 145.555 105.445) (width 0.3) (layer F.Cu) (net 27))
 (segment (start 144.92 107.62) (end 144.92 106.08) (width 0.3) (layer F.Cu) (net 27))
 (segment (start 152.75 94.329) (end 152.75 93.25) (width 0.2) (layer F.Cu) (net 27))
 (segment (start 152.159 94.92) (end 152.75 94.329) (width 0.2) (layer F.Cu) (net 27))
 (segment (start 145.555 94.92) (end 152.159 94.92) (width 0.2) (layer B.Cu) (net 27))
 (via (at 152.159 94.92) (size 0.5) (drill 0.3) (layers F.Cu B.Cu) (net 27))
 (segment (start 155.715 98.095) (end 157.62 96.19) (width 0.18) (layer F.Cu) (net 18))
 (segment (start 155.715 112.7) (end 155.715 98.095) (width 0.18) (layer F.Cu) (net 18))
 (segment (start 157.16 84.76) (end 157.62 85.22) (width 0.18) (layer F.Cu) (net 26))
 (segment (start 157.62 85.22) (end 157.62 86.03) (width 0.18) (layer F.Cu) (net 26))
 (segment (start 155.715 84.76) (end 157.16 84.76) (width 0.18) (layer F.Cu) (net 26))
 (via (at 144.8 105.1) (size 0.5) (drill 0.3) (layers F.Cu B.Cu) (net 30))
 (segment (start 144.85 105.15) (end 144.8 105.1) (width 0.18) (layer B.Cu) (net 30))
 (segment (start 148.65 105.15) (end 144.85 105.15) (width 0.18) (layer B.Cu) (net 30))
 (via (at 148.65 105.15) (size 0.5) (drill 0.3) (layers F.Cu B.Cu) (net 30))
 (segment (start 148.75 105.25) (end 148.75 106.75) (width 0.18) (layer F.Cu) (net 30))
 (segment (start 148.65 105.15) (end 148.75 105.25) (width 0.18) (layer F.Cu) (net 30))
 (segment (start 144.9 105) (end 144.8 105.1) (width 0.18) (layer F.Cu) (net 30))
 (segment (start 144.9 92.4) (end 144.9 105) (width 0.18) (layer F.Cu) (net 30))
 (segment (start 146.51 90.79) (end 144.9 92.4) (width 0.18) (layer F.Cu) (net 30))
 (segment (start 146.51 90.475) (end 146.51 90.79) (width 0.18) (layer F.Cu) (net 30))
 (segment (start 146.51 87.615) (end 146.51 90.475) (width 0.18) (layer F.Cu) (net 30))
 (segment (start 146.825 87.3) (end 146.51 87.615) (width 0.18) (layer F.Cu) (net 30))
 (segment (start 146.825 87.3) (end 155.715 87.3) (width 0.18) (layer B.Cu) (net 30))
 (via (at 146.825 87.3) (size 0.5) (drill 0.3) (layers F.Cu B.Cu) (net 30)))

